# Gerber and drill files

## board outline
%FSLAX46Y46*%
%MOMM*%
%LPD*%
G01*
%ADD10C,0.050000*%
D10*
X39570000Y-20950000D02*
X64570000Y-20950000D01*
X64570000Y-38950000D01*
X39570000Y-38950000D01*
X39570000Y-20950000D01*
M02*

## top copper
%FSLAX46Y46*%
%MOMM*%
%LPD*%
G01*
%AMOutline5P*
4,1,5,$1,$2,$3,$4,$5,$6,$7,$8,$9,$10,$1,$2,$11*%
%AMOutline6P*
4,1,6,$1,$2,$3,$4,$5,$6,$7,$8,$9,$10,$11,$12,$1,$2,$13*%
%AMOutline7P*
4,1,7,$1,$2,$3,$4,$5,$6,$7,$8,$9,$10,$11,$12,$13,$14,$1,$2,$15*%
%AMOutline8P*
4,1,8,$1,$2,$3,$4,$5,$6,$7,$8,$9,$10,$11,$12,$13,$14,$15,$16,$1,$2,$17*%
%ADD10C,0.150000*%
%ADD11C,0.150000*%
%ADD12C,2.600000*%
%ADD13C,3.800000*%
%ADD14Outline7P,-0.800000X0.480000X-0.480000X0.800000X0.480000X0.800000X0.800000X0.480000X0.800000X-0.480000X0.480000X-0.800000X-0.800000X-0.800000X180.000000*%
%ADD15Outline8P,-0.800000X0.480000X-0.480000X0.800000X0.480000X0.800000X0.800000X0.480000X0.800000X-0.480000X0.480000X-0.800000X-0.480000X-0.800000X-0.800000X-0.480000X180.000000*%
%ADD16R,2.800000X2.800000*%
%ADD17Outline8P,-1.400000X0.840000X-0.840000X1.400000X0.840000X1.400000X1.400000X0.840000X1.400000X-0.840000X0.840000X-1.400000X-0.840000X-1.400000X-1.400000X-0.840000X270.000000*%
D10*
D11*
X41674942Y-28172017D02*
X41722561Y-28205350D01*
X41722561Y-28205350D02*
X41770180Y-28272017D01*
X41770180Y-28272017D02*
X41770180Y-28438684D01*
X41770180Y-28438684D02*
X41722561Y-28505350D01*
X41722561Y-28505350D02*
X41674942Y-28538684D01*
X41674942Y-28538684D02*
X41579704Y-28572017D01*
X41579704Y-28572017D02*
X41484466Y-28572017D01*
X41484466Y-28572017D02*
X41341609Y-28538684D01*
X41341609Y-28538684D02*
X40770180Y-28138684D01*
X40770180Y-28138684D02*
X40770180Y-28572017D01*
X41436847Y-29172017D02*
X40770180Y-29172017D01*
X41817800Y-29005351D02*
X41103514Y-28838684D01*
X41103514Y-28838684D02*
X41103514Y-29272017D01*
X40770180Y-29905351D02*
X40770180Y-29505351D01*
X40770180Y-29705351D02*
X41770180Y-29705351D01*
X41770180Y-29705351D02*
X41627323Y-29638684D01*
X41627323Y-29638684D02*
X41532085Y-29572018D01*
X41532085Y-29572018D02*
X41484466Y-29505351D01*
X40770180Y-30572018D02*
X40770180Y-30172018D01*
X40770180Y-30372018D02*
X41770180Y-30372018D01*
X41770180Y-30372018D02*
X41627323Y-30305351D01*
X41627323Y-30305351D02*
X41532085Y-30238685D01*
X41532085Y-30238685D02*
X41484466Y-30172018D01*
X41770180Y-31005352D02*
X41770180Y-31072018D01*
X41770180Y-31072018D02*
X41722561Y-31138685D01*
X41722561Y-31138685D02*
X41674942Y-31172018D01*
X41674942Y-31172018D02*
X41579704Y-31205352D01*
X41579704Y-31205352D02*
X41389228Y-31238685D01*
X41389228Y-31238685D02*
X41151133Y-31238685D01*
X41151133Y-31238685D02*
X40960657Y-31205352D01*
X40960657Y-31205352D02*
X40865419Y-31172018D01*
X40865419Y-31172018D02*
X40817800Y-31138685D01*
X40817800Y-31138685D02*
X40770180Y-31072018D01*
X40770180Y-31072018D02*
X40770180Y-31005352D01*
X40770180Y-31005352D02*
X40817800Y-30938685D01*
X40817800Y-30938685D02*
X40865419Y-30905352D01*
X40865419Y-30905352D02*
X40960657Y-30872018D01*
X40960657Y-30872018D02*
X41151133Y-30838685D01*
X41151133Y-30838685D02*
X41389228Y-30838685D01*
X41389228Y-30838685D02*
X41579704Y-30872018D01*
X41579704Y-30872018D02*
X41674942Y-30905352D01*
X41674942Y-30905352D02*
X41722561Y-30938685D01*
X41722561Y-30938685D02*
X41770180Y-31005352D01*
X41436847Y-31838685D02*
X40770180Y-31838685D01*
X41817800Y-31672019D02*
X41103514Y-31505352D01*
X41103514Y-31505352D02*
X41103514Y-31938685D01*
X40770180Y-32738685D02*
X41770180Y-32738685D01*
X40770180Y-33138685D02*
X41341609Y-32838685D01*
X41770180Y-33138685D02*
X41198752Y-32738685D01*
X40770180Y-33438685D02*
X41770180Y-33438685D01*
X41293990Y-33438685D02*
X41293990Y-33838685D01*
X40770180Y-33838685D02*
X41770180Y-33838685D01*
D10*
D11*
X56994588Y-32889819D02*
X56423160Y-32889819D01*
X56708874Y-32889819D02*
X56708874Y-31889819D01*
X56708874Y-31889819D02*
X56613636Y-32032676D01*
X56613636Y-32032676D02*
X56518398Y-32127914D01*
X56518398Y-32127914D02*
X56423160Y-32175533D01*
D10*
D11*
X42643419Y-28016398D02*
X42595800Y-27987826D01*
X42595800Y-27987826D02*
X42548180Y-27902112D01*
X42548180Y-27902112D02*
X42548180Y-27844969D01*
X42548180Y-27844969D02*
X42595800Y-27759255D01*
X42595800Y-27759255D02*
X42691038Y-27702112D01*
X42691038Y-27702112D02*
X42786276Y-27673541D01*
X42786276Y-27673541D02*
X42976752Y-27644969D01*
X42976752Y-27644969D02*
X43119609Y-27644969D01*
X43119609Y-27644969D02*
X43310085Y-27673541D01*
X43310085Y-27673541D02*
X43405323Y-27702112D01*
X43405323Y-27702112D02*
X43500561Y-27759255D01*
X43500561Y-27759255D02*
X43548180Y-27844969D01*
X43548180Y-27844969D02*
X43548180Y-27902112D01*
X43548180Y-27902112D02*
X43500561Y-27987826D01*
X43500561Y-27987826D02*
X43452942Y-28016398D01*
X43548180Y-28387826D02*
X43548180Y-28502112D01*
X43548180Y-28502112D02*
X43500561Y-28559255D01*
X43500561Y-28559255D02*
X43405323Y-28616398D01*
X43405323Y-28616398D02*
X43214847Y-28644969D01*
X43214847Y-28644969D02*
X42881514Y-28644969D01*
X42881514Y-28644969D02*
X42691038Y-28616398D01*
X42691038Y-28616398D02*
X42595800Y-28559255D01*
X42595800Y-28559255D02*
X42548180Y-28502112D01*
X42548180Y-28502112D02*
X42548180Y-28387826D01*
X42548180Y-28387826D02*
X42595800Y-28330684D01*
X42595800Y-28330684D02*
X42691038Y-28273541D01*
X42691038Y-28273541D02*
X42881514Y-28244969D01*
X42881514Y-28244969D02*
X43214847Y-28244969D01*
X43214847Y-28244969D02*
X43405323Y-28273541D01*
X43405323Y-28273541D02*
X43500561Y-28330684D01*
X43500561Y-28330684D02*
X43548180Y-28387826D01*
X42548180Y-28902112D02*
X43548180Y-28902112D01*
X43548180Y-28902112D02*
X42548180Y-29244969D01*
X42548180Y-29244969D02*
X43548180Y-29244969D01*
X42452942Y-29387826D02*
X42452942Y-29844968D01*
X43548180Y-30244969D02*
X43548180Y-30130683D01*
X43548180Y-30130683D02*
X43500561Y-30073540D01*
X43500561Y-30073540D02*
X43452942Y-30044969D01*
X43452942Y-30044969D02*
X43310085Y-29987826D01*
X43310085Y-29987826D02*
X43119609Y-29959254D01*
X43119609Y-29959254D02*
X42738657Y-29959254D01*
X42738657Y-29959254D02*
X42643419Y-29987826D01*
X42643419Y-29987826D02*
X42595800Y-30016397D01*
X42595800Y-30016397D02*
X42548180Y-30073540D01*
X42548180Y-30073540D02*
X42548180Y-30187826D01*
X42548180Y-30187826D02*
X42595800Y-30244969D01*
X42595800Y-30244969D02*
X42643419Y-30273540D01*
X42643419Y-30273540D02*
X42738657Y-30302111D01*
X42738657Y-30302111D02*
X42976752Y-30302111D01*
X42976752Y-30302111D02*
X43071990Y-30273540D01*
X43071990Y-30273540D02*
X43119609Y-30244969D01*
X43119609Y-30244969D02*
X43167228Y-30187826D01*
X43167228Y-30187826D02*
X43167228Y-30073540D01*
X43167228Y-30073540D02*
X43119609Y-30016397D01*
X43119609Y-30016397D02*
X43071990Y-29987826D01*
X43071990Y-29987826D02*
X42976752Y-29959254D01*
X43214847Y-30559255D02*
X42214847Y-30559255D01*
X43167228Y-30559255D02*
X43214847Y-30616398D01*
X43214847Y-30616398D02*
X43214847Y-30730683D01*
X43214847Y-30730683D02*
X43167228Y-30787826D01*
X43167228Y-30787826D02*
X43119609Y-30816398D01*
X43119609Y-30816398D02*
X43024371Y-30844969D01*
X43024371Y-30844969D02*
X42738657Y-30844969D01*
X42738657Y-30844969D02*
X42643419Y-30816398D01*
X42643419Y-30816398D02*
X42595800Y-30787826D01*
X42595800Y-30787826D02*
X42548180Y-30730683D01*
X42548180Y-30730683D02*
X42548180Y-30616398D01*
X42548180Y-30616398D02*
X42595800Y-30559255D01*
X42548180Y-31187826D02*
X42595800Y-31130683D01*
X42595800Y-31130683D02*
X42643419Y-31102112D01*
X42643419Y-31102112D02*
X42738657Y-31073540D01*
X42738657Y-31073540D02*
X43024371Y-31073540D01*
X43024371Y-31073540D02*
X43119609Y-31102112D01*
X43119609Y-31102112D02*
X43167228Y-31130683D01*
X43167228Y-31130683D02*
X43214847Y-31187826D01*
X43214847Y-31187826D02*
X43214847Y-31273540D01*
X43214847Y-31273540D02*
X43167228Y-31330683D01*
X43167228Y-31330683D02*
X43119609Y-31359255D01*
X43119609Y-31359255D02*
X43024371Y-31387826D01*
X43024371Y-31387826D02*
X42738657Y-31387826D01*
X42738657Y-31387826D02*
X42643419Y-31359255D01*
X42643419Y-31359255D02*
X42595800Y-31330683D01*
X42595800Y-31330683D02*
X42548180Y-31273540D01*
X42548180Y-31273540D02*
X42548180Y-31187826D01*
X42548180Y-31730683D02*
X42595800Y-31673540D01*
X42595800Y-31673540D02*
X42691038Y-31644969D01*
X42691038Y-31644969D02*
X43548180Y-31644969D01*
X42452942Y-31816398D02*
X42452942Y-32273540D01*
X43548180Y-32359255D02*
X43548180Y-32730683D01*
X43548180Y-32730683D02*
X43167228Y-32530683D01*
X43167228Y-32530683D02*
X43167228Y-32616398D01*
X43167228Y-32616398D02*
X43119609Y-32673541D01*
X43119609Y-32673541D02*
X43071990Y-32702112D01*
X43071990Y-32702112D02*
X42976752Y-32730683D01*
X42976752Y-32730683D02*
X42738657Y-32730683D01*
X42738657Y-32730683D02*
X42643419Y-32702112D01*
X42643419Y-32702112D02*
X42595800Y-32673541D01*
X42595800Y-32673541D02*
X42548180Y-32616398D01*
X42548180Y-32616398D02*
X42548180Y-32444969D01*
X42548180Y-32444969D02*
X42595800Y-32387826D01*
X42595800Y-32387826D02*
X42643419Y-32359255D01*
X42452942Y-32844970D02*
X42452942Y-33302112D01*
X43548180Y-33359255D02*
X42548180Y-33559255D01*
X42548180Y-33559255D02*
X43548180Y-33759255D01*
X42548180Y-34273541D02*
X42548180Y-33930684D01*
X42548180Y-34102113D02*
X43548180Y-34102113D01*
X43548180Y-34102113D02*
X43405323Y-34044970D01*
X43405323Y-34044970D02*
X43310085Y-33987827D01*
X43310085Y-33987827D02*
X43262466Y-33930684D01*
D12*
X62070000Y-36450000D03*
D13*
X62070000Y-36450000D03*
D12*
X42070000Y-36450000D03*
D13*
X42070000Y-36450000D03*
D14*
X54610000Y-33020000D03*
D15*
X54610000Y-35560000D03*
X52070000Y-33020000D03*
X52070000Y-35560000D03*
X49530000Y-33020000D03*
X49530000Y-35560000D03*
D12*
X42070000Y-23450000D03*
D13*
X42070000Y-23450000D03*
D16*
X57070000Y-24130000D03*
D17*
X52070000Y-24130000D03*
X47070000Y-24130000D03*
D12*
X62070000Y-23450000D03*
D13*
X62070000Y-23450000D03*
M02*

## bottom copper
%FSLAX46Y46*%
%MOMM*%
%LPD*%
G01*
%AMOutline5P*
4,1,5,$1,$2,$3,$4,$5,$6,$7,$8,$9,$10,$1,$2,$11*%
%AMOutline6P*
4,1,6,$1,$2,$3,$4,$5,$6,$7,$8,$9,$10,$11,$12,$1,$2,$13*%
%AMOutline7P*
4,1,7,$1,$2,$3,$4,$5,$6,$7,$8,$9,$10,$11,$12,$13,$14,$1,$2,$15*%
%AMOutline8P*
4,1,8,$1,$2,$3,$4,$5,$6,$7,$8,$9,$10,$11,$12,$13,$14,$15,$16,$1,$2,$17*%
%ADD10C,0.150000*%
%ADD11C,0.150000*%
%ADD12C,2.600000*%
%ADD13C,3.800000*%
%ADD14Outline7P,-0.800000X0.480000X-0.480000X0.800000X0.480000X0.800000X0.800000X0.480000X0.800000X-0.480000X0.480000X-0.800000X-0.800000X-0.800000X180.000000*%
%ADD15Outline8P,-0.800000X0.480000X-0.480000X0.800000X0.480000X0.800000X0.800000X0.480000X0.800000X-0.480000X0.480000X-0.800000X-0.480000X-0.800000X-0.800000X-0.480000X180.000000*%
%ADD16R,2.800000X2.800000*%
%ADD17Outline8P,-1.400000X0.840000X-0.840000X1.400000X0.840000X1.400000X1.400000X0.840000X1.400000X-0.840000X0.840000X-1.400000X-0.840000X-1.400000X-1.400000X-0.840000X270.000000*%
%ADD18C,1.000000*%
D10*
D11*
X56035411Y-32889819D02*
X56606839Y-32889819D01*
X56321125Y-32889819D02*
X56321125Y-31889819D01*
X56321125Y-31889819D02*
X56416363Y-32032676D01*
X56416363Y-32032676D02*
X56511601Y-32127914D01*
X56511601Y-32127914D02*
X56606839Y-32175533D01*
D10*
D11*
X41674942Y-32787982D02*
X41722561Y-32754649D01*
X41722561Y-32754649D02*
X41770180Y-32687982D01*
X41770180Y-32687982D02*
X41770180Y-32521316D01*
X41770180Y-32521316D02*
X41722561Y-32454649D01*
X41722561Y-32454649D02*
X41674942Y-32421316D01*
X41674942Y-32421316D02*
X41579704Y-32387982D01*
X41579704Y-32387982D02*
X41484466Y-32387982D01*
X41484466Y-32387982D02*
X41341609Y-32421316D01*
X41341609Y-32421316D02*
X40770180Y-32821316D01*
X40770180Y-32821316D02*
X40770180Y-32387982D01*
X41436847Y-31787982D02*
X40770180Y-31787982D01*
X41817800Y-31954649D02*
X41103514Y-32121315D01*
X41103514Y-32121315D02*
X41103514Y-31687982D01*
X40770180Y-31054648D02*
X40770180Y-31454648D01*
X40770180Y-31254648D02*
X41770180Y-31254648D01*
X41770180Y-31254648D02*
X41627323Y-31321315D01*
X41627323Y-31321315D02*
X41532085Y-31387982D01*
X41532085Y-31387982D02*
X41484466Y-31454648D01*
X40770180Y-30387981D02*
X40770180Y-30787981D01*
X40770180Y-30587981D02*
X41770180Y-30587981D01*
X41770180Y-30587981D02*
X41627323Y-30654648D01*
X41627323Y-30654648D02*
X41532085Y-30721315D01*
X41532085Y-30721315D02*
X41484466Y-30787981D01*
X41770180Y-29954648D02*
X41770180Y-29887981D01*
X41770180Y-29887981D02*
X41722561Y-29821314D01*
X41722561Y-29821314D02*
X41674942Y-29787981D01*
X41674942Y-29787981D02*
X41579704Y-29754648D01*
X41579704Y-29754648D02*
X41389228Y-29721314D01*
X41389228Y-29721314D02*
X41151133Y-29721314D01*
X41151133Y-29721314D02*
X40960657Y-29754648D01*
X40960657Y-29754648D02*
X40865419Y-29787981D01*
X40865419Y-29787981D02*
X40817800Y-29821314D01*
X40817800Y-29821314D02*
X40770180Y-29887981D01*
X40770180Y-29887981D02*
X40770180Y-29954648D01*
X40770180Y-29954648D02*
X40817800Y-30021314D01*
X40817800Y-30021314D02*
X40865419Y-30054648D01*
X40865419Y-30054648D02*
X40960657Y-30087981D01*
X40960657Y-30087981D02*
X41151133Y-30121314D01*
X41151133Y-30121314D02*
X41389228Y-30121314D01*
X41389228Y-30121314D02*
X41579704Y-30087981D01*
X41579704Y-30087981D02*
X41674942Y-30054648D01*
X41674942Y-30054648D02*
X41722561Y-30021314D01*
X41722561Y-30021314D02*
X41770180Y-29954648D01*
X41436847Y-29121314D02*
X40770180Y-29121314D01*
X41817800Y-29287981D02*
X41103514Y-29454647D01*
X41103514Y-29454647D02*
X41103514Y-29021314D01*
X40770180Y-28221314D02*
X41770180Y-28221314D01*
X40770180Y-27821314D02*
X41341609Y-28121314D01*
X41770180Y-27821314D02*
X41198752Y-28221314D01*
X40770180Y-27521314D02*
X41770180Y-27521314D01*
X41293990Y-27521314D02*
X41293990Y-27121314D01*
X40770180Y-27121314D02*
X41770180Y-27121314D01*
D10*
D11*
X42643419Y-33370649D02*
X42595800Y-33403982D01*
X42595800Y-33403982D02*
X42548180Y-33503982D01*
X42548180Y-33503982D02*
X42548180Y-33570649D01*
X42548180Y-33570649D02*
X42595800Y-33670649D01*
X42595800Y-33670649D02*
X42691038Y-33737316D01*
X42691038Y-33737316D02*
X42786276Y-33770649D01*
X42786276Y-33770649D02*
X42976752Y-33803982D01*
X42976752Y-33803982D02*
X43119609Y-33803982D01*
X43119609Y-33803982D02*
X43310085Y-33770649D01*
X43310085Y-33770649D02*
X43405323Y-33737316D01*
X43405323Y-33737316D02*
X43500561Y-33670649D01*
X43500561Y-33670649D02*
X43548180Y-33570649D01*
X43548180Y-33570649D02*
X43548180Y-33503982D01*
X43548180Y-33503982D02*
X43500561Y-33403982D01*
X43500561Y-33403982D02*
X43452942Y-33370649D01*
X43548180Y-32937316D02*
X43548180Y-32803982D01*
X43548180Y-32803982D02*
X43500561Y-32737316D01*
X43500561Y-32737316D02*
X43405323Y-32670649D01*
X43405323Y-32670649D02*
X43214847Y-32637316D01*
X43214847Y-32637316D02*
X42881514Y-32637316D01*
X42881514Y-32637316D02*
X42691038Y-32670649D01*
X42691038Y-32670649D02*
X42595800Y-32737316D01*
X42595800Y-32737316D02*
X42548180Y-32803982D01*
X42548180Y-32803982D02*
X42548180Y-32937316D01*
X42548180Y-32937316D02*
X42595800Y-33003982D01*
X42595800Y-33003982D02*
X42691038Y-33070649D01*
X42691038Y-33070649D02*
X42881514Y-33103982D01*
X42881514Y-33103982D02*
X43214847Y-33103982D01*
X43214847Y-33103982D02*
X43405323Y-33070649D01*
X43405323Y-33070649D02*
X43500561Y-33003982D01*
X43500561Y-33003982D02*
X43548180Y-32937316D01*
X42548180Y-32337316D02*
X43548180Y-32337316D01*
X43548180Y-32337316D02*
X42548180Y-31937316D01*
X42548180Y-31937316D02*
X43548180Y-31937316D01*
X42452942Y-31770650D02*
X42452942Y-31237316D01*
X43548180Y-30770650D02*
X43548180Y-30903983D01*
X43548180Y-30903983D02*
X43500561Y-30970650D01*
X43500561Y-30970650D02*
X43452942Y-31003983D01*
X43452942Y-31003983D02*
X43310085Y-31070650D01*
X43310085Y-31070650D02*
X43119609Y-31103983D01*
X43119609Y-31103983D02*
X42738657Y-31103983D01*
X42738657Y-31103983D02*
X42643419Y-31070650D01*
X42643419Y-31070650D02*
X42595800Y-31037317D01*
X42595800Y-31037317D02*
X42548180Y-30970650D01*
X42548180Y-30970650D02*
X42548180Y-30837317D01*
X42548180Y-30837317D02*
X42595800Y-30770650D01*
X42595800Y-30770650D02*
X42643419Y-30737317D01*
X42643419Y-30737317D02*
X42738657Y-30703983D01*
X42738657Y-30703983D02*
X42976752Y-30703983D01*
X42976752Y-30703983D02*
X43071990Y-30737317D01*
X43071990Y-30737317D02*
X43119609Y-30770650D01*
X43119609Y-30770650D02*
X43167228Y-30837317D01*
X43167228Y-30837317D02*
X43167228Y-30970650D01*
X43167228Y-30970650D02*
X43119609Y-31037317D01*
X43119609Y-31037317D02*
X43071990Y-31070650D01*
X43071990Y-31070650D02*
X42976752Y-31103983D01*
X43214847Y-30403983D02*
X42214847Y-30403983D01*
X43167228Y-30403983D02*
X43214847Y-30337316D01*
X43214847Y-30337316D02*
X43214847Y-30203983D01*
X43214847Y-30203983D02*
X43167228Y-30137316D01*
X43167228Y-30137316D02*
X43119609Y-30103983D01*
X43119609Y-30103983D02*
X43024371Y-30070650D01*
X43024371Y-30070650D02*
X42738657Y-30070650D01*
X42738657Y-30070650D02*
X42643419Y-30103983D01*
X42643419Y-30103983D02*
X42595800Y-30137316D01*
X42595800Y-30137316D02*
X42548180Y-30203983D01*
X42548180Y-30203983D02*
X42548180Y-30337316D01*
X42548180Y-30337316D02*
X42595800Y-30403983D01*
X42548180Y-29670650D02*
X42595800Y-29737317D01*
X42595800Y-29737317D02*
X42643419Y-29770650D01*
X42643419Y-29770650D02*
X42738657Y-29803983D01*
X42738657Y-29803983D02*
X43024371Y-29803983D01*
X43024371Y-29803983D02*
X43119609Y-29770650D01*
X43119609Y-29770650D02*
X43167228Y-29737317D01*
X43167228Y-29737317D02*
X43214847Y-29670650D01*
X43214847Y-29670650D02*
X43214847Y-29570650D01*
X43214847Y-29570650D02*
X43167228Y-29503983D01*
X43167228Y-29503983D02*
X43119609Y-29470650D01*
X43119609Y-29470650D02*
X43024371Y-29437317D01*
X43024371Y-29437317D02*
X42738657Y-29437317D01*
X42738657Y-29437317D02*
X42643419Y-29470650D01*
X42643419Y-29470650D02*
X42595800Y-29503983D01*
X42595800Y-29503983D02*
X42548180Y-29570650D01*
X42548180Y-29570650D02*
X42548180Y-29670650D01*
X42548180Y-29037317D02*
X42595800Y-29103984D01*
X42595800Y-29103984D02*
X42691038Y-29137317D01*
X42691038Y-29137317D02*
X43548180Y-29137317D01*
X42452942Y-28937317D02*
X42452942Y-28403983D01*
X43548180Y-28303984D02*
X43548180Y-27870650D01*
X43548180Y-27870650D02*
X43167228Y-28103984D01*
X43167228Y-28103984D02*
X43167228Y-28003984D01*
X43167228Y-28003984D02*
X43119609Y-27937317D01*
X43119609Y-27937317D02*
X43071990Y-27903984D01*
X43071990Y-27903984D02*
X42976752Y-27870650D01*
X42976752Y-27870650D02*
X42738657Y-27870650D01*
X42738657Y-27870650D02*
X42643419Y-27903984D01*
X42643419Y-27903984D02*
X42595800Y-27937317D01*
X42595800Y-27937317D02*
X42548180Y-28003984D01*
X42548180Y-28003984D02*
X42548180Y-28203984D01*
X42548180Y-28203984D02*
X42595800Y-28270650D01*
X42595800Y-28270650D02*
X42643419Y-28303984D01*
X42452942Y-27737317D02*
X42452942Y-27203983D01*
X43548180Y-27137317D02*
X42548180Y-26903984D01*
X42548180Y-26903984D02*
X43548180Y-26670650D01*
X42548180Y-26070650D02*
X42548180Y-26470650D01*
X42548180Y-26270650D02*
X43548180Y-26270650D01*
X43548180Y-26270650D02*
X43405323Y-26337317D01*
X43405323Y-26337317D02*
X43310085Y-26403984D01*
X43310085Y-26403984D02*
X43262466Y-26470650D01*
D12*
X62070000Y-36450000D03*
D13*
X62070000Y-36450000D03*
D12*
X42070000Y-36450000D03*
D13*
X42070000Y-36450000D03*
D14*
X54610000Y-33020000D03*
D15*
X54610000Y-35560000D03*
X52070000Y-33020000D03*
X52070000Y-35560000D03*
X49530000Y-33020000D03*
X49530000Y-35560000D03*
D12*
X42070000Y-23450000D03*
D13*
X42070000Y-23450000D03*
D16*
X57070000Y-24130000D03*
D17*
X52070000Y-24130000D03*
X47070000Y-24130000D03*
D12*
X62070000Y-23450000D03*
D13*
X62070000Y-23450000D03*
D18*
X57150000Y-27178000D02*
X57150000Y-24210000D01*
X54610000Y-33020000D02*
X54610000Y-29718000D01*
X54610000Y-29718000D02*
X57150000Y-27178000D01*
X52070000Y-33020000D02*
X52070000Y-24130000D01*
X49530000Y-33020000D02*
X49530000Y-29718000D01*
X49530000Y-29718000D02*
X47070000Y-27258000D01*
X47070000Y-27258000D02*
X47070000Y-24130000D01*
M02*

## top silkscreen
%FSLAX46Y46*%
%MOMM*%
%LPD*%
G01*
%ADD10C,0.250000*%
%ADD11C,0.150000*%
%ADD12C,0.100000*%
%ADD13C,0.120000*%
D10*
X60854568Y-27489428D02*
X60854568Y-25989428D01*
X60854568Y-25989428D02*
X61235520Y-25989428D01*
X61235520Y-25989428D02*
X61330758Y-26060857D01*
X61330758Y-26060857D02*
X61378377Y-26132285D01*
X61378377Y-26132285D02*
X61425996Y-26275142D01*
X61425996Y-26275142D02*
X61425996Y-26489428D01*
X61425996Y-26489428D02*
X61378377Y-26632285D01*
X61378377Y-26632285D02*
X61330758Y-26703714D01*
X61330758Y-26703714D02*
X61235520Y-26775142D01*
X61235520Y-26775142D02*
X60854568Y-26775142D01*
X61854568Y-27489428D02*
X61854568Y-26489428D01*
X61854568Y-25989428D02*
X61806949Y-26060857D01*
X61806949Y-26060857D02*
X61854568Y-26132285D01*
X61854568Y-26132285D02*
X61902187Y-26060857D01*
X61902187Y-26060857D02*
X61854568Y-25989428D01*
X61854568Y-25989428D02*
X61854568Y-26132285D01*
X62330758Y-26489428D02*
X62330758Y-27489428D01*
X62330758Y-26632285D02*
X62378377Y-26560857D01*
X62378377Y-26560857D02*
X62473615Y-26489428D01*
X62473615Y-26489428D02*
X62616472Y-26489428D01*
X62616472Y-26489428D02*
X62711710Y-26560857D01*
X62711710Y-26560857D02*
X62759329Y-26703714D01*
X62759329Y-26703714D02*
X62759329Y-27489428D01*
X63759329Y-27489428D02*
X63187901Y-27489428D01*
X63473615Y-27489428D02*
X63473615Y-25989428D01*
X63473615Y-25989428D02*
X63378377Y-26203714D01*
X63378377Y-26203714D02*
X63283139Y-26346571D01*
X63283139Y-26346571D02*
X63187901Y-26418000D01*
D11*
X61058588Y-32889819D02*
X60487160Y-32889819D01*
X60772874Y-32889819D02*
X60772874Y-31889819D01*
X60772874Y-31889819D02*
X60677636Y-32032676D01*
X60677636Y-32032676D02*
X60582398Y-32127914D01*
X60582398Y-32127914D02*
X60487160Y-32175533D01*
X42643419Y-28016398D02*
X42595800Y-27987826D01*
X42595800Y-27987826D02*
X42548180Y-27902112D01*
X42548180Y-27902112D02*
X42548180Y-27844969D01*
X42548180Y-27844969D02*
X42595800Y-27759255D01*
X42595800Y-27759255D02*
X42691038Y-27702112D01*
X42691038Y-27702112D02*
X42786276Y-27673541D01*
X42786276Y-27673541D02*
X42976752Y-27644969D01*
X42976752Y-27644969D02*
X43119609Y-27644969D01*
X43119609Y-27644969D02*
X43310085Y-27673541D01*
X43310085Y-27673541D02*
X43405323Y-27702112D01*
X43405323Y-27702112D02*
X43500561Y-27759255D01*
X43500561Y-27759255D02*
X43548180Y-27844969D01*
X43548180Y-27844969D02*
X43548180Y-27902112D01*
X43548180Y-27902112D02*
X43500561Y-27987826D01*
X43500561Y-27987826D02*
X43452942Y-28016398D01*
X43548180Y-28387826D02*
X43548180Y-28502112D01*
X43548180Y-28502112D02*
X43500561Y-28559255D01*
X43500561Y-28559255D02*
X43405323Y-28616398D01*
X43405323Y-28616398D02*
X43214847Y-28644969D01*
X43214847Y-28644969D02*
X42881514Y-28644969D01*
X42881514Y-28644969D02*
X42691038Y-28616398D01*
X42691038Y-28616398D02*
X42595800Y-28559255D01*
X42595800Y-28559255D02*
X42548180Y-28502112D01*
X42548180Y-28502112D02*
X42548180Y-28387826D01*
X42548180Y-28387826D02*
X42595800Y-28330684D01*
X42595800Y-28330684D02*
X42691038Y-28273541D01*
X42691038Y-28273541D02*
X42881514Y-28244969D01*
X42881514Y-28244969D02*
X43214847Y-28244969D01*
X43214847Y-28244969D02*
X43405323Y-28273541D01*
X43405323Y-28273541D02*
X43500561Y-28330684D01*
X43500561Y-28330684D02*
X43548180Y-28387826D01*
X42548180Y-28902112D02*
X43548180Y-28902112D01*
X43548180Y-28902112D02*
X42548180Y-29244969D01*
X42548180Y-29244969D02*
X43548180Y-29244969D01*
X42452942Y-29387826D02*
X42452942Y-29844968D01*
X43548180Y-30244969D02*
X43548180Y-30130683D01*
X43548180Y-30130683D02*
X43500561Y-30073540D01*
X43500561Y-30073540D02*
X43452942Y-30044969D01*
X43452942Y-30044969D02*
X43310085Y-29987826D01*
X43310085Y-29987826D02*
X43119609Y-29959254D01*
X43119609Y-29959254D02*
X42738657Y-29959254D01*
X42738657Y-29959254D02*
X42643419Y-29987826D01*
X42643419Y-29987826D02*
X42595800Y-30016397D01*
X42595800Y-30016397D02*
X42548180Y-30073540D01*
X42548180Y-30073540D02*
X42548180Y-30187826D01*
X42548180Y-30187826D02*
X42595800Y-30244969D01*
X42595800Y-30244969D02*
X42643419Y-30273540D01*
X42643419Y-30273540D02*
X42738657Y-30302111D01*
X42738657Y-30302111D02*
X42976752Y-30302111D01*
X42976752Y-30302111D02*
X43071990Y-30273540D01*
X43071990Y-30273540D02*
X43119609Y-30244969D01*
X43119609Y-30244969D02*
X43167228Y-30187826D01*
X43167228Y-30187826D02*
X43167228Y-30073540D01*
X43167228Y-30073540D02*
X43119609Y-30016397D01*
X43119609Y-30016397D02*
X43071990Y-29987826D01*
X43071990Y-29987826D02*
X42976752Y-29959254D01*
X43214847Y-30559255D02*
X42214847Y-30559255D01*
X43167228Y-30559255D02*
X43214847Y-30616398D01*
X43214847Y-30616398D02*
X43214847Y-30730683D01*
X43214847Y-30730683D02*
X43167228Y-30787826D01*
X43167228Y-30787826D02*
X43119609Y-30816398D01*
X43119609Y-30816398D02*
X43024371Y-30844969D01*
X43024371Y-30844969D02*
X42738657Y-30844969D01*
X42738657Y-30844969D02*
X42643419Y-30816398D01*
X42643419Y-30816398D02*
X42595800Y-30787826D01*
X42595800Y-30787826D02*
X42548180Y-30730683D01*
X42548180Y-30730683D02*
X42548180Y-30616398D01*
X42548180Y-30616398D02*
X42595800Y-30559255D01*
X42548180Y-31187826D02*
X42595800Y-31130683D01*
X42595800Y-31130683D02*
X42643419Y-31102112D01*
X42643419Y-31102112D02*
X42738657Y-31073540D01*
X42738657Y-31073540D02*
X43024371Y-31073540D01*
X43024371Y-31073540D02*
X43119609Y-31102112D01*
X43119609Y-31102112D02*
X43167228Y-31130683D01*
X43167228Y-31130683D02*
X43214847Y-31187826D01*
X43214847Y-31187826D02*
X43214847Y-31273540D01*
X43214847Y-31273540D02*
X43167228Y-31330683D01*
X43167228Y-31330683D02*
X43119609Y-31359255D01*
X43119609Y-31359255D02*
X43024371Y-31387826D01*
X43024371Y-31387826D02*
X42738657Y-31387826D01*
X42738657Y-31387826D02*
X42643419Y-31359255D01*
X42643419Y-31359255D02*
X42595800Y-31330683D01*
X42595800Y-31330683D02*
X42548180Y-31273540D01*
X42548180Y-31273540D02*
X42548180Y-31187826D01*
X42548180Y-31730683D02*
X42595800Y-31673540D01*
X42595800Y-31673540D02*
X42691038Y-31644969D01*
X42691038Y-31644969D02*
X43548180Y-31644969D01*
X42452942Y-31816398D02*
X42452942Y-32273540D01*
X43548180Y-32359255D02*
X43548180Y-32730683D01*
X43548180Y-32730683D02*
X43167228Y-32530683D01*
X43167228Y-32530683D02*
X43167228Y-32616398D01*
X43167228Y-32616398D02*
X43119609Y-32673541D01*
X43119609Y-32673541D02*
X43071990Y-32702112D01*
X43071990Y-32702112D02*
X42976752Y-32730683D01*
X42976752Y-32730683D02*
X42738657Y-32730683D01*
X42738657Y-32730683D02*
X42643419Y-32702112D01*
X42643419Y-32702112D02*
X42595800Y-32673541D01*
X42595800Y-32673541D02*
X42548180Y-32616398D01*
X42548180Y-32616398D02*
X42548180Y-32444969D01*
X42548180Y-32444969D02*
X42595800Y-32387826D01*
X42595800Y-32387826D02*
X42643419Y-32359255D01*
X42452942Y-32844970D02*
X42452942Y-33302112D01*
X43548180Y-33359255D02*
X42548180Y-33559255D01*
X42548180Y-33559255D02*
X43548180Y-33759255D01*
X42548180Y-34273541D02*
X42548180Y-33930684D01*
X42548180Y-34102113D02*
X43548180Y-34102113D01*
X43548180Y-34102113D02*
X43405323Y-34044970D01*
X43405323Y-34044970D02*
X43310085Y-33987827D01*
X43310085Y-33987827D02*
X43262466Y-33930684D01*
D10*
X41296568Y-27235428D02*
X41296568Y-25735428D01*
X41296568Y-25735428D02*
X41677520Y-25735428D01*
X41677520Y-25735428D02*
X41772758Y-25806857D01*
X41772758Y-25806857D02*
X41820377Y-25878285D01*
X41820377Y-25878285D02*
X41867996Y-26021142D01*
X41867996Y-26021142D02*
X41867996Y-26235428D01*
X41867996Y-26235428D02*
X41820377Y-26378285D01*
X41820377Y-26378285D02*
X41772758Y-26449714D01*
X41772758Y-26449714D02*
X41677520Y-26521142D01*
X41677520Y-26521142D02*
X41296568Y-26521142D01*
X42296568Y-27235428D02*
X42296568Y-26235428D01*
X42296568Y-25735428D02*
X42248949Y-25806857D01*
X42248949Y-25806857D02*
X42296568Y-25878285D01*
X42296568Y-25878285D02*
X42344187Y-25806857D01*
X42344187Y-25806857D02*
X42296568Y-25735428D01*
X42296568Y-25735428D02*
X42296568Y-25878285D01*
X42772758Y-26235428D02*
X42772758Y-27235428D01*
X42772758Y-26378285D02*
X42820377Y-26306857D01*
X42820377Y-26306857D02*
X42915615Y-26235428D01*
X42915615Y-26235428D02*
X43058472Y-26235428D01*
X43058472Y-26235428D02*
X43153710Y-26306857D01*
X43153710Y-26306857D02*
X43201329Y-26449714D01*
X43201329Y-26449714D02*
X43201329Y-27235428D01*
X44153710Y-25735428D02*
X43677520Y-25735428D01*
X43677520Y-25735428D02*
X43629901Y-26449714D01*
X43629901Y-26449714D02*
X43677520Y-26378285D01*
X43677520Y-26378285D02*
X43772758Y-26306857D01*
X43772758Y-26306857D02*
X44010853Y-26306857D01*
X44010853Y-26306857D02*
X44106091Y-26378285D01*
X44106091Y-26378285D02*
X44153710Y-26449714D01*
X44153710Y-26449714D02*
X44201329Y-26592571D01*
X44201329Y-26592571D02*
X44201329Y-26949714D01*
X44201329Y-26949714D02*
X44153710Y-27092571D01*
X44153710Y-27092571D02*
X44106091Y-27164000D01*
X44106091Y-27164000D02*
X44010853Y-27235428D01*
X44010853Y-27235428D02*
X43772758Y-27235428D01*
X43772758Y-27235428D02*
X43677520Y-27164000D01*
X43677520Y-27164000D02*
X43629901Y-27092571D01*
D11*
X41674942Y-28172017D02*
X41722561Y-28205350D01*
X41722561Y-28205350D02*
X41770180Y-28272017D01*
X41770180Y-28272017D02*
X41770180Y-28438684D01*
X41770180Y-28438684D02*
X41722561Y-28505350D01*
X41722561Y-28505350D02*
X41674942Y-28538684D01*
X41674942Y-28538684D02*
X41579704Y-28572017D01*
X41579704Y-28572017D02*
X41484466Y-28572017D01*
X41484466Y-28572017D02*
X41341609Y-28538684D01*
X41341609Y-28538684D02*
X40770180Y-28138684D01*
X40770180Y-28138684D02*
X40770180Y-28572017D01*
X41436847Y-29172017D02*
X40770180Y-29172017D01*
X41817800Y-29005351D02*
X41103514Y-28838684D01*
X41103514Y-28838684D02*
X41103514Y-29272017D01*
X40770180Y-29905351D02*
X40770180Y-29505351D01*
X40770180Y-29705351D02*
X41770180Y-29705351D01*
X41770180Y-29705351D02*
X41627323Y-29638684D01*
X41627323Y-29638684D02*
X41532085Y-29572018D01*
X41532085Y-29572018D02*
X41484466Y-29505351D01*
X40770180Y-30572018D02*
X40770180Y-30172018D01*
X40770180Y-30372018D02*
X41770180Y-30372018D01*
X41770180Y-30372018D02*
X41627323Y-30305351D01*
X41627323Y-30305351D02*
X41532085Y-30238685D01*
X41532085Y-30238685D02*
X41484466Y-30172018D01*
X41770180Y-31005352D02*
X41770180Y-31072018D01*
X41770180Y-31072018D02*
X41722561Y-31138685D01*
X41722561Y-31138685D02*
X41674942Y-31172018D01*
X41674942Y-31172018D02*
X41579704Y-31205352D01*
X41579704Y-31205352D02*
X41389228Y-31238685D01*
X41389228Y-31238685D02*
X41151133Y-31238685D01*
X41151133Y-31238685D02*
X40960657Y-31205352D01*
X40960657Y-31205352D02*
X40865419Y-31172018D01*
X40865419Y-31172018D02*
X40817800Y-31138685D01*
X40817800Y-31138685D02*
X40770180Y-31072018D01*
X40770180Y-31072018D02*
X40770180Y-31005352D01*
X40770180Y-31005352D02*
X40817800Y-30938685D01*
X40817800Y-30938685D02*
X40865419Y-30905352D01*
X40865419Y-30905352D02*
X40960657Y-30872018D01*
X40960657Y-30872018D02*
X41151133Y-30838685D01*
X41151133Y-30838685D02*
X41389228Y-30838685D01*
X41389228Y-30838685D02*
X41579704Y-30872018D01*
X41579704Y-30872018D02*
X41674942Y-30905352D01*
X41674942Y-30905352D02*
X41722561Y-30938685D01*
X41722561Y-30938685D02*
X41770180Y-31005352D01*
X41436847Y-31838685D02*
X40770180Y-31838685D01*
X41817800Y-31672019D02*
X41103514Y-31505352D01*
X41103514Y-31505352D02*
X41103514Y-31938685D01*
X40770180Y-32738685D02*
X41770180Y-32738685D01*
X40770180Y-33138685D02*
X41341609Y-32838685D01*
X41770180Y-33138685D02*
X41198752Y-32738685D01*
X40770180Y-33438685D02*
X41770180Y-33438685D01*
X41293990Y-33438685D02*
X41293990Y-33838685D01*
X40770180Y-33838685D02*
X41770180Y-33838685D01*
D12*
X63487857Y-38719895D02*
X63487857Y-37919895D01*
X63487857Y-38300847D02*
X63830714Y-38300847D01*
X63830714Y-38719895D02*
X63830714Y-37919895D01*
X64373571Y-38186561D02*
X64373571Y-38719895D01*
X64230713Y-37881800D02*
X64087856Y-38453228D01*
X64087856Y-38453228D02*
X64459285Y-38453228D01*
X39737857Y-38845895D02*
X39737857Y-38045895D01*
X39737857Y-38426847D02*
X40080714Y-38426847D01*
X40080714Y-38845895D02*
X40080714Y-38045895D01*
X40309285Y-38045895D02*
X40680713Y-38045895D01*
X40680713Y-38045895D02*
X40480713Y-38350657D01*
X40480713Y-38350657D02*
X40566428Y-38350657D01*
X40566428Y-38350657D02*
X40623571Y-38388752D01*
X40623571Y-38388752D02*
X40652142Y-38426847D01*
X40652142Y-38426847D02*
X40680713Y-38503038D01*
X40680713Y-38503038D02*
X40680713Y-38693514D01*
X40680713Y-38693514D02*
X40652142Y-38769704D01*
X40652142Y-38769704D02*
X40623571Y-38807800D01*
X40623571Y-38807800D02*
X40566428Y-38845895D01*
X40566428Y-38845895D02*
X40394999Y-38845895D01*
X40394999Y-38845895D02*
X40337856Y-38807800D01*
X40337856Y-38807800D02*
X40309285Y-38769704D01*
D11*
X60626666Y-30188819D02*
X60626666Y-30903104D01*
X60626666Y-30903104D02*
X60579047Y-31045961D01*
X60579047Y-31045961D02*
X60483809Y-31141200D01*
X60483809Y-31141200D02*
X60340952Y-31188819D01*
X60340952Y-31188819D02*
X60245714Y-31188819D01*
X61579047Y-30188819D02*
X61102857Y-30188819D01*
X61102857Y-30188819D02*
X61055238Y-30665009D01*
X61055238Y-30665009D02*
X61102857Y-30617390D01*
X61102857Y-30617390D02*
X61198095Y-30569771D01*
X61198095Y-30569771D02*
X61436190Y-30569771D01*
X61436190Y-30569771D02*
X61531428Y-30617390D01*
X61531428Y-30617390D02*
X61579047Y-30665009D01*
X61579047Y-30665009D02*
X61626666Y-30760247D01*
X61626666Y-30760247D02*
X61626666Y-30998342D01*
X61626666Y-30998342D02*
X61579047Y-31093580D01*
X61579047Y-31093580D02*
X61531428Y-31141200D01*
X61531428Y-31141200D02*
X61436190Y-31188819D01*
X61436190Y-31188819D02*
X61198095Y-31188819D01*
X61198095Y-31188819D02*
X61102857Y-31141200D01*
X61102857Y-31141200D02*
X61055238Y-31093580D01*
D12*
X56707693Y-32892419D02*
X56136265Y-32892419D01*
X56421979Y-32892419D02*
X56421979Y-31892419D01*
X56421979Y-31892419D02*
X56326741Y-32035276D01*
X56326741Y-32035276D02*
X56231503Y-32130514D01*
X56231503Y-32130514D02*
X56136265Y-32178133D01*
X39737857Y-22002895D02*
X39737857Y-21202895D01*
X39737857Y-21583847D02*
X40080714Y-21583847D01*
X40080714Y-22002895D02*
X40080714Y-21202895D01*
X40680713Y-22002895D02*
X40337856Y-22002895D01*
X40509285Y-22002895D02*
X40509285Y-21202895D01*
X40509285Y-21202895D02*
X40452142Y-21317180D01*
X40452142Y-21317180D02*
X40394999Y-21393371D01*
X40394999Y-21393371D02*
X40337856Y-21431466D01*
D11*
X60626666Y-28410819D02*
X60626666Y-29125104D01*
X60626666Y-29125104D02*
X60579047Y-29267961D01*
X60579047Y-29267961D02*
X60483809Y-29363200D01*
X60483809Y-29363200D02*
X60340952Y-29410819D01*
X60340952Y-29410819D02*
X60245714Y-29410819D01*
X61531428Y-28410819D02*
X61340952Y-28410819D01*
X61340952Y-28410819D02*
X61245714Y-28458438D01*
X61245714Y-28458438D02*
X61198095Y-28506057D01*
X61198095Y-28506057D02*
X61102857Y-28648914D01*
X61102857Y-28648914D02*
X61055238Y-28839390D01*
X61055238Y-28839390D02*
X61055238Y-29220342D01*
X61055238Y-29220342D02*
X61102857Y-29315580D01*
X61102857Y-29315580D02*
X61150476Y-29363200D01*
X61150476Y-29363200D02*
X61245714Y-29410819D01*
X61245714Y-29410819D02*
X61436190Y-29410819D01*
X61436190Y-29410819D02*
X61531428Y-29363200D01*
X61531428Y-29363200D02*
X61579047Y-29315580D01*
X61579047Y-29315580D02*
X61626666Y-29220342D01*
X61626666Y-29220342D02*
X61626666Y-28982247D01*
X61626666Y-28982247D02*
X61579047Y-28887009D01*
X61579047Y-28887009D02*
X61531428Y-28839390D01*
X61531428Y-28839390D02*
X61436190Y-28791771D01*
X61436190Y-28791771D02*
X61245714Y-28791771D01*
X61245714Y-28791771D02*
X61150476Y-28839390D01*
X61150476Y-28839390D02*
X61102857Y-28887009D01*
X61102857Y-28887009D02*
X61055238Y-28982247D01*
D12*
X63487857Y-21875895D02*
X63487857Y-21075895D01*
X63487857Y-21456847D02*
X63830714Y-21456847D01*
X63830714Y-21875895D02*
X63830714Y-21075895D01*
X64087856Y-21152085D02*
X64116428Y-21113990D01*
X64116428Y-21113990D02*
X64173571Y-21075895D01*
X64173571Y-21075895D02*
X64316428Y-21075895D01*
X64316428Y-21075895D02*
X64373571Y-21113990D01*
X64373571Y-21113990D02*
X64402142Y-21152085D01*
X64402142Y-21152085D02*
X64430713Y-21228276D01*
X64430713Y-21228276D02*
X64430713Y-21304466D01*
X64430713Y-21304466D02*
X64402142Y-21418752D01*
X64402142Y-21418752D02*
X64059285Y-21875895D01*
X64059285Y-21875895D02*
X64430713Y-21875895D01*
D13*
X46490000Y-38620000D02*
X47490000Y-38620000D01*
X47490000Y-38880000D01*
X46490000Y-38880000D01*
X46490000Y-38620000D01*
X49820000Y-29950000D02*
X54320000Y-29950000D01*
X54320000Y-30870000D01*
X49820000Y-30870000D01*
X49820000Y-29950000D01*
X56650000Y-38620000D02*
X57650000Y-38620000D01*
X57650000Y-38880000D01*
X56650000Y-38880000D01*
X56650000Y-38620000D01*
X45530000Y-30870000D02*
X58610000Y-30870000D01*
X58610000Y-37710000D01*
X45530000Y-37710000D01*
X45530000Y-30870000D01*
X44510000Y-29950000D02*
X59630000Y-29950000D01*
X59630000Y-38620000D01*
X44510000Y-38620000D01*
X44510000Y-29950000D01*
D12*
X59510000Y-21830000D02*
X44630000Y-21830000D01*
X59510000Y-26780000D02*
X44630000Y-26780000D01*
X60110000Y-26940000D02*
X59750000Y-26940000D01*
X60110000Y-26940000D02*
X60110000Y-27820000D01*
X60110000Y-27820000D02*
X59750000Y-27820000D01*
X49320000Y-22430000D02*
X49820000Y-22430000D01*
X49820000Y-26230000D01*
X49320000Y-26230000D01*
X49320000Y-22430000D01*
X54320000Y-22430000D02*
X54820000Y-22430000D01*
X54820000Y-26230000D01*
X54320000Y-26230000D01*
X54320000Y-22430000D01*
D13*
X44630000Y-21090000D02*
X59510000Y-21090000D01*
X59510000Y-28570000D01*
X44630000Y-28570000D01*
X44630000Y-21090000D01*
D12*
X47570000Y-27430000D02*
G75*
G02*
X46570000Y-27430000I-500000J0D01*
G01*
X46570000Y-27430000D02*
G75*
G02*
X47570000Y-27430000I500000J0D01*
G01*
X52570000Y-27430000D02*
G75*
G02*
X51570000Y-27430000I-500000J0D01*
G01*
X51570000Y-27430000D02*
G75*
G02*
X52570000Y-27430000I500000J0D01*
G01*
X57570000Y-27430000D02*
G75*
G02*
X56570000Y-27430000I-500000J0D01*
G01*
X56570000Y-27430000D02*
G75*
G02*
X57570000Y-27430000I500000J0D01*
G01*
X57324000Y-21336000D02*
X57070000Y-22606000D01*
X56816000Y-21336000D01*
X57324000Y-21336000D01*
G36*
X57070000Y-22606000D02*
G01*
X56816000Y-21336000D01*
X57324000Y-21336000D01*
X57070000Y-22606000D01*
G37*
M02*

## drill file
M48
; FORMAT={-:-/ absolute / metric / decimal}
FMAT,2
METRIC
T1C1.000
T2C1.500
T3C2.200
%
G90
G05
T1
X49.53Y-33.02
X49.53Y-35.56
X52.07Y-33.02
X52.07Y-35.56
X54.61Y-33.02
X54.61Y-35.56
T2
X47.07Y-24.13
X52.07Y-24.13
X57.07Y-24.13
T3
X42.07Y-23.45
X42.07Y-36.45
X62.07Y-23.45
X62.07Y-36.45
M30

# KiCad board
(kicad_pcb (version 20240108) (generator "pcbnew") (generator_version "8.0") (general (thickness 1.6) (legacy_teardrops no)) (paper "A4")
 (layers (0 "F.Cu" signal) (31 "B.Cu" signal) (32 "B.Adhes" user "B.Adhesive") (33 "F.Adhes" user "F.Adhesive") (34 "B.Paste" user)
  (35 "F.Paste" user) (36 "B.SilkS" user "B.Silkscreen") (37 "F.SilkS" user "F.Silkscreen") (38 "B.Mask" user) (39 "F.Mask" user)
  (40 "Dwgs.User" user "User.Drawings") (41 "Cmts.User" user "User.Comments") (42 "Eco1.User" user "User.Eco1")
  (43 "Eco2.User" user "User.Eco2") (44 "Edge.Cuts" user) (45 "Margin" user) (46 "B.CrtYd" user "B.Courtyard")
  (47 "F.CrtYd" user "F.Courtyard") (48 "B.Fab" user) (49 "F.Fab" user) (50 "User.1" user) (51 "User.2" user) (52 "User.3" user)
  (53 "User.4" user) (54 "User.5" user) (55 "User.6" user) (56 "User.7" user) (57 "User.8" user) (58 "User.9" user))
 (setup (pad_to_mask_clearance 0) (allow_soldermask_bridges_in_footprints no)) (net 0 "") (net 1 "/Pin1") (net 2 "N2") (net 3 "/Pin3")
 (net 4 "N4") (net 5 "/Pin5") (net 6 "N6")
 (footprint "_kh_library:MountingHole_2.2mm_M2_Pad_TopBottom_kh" (layer "F.Cu") (at 62.07 36.45)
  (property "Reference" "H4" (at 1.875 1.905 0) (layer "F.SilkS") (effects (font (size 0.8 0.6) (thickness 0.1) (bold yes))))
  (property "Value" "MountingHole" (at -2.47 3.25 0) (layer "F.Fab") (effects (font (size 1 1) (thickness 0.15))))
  (pad "1" thru_hole circle (at 0 0) (size 2.6 2.6) (drill 2.2) (layers "*.Cu" "*.Mask") (remove_unused_layers no))
  (pad "1" connect circle (at 0 0) (size 3.8 3.8) (layers "F.Cu" "F.Mask"))
  (pad "1" connect circle (at 0 0) (size 3.8 3.8) (layers "B.Cu" "B.Mask")))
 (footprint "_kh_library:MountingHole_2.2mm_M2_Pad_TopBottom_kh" (layer "F.Cu") (at 42.07 36.45)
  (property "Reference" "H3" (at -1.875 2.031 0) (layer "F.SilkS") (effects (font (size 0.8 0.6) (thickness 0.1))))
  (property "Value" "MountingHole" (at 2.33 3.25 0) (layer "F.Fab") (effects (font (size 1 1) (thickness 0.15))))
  (pad "1" thru_hole circle (at 0 0) (size 2.6 2.6) (drill 2.2) (layers "*.Cu" "*.Mask") (remove_unused_layers no))
  (pad "1" connect circle (at 0 0) (size 3.8 3.8) (layers "F.Cu" "F.Mask"))
  (pad "1" connect circle (at 0 0) (size 3.8 3.8) (layers "B.Cu" "B.Mask")))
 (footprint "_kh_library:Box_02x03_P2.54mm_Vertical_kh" (layer "F.Cu") (at 54.61 33.02 180)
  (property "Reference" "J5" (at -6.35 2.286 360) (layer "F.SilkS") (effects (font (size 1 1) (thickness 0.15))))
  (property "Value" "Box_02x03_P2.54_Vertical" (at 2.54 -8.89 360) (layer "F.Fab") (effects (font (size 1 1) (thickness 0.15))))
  (fp_rect (start 7.12 -5.6) (end 8.12 -5.86) (stroke (width 0.12) (type default)) (fill none) (layer "F.SilkS"))
  (fp_rect (start 0.29 3.07) (end 4.79 2.15) (stroke (width 0.12) (type default)) (fill none) (layer "F.SilkS"))
  (fp_rect (start -3.04 -5.6) (end -2.04 -5.86) (stroke (width 0.12) (type default)) (fill none) (layer "F.SilkS"))
  (fp_rect (start -4 2.15) (end 9.08 -4.69) (stroke (width 0.12) (type default)) (fill none) (layer "F.SilkS"))
  (fp_rect (start -5.02 3.07) (end 10.1 -5.6) (stroke (width 0.12) (type default)) (fill none) (layer "F.SilkS"))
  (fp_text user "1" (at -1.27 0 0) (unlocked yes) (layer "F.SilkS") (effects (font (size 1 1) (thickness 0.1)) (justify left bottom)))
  (pad "1" thru_hole roundrect (at 0 0 180) (size 1.6 1.6) (drill 1) (layers "*.Cu" "*.Mask") (remove_unused_layers no) (roundrect_rratio 0)
   (chamfer_ratio 0.2) (chamfer top_left top_right bottom_right) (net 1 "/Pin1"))
  (pad "2" thru_hole roundrect (at 0 -2.54 180) (size 1.6 1.6) (drill 1) (layers "*.Cu" "*.Mask") (remove_unused_layers no)
   (roundrect_rratio 0) (chamfer_ratio 0.2) (chamfer top_left top_right bottom_left bottom_right) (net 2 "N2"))
  (pad "3" thru_hole roundrect (at 2.54 0 180) (size 1.6 1.6) (drill 1) (layers "*.Cu" "*.Mask") (remove_unused_layers no)
   (roundrect_rratio 0) (chamfer_ratio 0.2) (chamfer top_left top_right bottom_left bottom_right) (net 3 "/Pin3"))
  (pad "4" thru_hole roundrect (at 2.54 -2.54 180) (size 1.6 1.6) (drill 1) (layers "*.Cu" "*.Mask") (remove_unused_layers no)
   (roundrect_rratio 0) (chamfer_ratio 0.2) (chamfer top_left top_right bottom_left bottom_right) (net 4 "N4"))
  (pad "5" thru_hole roundrect (at 5.08 0 180) (size 1.6 1.6) (drill 1) (layers "*.Cu" "*.Mask") (remove_unused_layers no)
   (roundrect_rratio 0) (chamfer_ratio 0.2) (chamfer top_left top_right bottom_left bottom_right) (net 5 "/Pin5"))
  (pad "6" thru_hole roundrect (at 5.08 -2.54 180) (size 1.6 1.6) (drill 1) (layers "*.Cu" "*.Mask") (remove_unused_layers no)
   (roundrect_rratio 0) (chamfer_ratio 0.2) (chamfer top_left top_right bottom_left bottom_right) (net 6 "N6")))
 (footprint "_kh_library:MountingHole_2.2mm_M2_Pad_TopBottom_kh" (layer "F.Cu") (at 42.07 23.45)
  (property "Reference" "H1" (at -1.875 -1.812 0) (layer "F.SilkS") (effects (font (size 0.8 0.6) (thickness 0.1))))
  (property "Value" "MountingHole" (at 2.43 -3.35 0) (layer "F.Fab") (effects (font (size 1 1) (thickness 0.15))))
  (pad "1" thru_hole circle (at 0 0) (size 2.6 2.6) (drill 2.2) (layers "*.Cu" "*.Mask") (remove_unused_layers no))
  (pad "1" connect circle (at 0 0) (size 3.8 3.8) (layers "F.Cu" "F.Mask"))
  (pad "1" connect circle (at 0 0) (size 3.8 3.8) (layers "B.Cu" "B.Mask")))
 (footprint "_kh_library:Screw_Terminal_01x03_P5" (layer "F.Cu") (at 57.07 24.13 -90)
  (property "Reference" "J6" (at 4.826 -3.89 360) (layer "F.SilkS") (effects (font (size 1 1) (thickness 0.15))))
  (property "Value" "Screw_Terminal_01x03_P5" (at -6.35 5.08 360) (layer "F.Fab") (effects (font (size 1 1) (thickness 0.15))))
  (fp_line (start -2.3 -2.44) (end -2.3 12.44) (stroke (width 0.1) (type default)) (layer "F.SilkS"))
  (fp_line (start 2.65 -2.44) (end 2.65 12.44) (stroke (width 0.1) (type default)) (layer "F.SilkS"))
  (fp_line (start 2.81 -3.04) (end 2.81 -2.68) (stroke (width 0.1) (type default)) (layer "F.SilkS"))
  (fp_line (start 2.81 -3.04) (end 3.69 -3.04) (stroke (width 0.1) (type default)) (layer "F.SilkS"))
  (fp_line (start 3.69 -3.04) (end 3.69 -2.68) (stroke (width 0.1) (type default)) (layer "F.SilkS"))
  (fp_rect (start -1.7 7.25) (end 2.1 7.75) (stroke (width 0.1) (type default)) (fill none) (layer "F.SilkS"))
  (fp_rect (start -1.7 2.25) (end 2.1 2.75) (stroke (width 0.1) (type default)) (fill none) (layer "F.SilkS"))
  (fp_rect (start -3.04 -2.44) (end 4.44 12.44) (stroke (width 0.12) (type default)) (fill none) (layer "F.SilkS"))
  (fp_circle (center 3.3 10) (end 3.8 10) (stroke (width 0.1) (type default)) (fill none) (layer "F.SilkS"))
  (fp_circle (center 3.3 5) (end 3.8 5) (stroke (width 0.1) (type default)) (fill none) (layer "F.SilkS"))
  (fp_circle (center 3.3 0) (end 3.8 0) (stroke (width 0.1) (type default)) (fill none) (layer "F.SilkS"))
  (fp_poly (pts (xy -2.794 -0.254) (xy -1.524 0) (xy -2.794 0.254)) (stroke (width 0.1) (type solid)) (fill solid) (layer "F.SilkS"))
  (pad "1" thru_hole rect (at 0 0 270) (size 2.8 2.8) (drill 1.5) (layers "*.Cu" "*.Mask") (remove_unused_layers no) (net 1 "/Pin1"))
  (pad "2" thru_hole roundrect (at 0 5 270) (size 2.8 2.8) (drill 1.5) (layers "*.Cu" "*.Mask") (remove_unused_layers no)
   (roundrect_rratio 0) (chamfer_ratio 0.2) (chamfer top_left top_right bottom_left bottom_right) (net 3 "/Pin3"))
  (pad "3" thru_hole roundrect (at 0 10 270) (size 2.8 2.8) (drill 1.5) (layers "*.Cu" "*.Mask") (remove_unused_layers no)
   (roundrect_rratio 0) (chamfer_ratio 0.2) (chamfer top_left top_right bottom_left bottom_right) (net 5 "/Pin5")))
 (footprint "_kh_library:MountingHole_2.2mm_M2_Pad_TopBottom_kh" (layer "F.Cu") (at 62.07 23.45)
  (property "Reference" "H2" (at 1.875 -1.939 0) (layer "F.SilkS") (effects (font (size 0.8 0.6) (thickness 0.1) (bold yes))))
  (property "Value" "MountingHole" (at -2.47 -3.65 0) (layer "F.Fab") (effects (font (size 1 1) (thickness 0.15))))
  (pad "1" thru_hole circle (at 0 0) (size 2.6 2.6) (drill 2.2) (layers "*.Cu" "*.Mask") (remove_unused_layers no))
  (pad "1" connect circle (at 0 0) (size 3.8 3.8) (layers "F.Cu" "F.Mask"))
  (pad "1" connect circle (at 0 0) (size 3.8 3.8) (layers "B.Cu" "B.Mask")))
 (gr_rect (start 39.57 20.95) (end 64.57 38.95) (stroke (width 0.05) (type default)) (fill none) (layer "Edge.Cuts"))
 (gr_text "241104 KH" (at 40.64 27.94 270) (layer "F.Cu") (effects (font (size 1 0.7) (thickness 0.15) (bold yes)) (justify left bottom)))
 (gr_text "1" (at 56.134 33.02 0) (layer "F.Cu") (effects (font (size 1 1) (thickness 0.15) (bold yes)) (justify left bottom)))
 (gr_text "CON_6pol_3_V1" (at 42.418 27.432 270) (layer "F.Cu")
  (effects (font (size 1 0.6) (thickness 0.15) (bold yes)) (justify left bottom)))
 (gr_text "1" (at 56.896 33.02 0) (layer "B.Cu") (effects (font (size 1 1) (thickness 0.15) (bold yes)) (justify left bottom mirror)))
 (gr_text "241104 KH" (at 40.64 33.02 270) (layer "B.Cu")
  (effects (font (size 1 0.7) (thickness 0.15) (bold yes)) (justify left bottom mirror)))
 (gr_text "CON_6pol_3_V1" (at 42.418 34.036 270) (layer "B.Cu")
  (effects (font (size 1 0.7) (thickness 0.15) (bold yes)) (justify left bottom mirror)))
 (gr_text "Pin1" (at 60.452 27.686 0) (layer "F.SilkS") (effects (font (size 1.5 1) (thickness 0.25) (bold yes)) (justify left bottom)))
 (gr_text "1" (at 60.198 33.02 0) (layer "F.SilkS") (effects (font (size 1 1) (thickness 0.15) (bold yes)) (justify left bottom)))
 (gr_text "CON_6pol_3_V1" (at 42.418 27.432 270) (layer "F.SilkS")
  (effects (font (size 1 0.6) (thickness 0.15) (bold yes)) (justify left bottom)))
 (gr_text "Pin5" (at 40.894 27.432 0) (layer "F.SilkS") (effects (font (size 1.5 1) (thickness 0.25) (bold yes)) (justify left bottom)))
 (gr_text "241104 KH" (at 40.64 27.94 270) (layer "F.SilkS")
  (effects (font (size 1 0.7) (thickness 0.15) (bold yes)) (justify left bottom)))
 (segment (start 57.15 27.178) (end 57.15 24.21) (width 1) (layer "B.Cu") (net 1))
 (segment (start 54.61 33.02) (end 54.61 29.718) (width 1) (layer "B.Cu") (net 1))
 (segment (start 54.61 29.718) (end 57.15 27.178) (width 1) (layer "B.Cu") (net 1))
 (segment (start 52.07 33.02) (end 52.07 24.13) (width 1) (layer "B.Cu") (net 3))
 (segment (start 49.53 33.02) (end 49.53 29.718) (width 1) (layer "B.Cu") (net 5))
 (segment (start 49.53 29.718) (end 47.07 27.258) (width 1) (layer "B.Cu") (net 5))
 (segment (start 47.07 27.258) (end 47.07 24.13) (width 1) (layer "B.Cu") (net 5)))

